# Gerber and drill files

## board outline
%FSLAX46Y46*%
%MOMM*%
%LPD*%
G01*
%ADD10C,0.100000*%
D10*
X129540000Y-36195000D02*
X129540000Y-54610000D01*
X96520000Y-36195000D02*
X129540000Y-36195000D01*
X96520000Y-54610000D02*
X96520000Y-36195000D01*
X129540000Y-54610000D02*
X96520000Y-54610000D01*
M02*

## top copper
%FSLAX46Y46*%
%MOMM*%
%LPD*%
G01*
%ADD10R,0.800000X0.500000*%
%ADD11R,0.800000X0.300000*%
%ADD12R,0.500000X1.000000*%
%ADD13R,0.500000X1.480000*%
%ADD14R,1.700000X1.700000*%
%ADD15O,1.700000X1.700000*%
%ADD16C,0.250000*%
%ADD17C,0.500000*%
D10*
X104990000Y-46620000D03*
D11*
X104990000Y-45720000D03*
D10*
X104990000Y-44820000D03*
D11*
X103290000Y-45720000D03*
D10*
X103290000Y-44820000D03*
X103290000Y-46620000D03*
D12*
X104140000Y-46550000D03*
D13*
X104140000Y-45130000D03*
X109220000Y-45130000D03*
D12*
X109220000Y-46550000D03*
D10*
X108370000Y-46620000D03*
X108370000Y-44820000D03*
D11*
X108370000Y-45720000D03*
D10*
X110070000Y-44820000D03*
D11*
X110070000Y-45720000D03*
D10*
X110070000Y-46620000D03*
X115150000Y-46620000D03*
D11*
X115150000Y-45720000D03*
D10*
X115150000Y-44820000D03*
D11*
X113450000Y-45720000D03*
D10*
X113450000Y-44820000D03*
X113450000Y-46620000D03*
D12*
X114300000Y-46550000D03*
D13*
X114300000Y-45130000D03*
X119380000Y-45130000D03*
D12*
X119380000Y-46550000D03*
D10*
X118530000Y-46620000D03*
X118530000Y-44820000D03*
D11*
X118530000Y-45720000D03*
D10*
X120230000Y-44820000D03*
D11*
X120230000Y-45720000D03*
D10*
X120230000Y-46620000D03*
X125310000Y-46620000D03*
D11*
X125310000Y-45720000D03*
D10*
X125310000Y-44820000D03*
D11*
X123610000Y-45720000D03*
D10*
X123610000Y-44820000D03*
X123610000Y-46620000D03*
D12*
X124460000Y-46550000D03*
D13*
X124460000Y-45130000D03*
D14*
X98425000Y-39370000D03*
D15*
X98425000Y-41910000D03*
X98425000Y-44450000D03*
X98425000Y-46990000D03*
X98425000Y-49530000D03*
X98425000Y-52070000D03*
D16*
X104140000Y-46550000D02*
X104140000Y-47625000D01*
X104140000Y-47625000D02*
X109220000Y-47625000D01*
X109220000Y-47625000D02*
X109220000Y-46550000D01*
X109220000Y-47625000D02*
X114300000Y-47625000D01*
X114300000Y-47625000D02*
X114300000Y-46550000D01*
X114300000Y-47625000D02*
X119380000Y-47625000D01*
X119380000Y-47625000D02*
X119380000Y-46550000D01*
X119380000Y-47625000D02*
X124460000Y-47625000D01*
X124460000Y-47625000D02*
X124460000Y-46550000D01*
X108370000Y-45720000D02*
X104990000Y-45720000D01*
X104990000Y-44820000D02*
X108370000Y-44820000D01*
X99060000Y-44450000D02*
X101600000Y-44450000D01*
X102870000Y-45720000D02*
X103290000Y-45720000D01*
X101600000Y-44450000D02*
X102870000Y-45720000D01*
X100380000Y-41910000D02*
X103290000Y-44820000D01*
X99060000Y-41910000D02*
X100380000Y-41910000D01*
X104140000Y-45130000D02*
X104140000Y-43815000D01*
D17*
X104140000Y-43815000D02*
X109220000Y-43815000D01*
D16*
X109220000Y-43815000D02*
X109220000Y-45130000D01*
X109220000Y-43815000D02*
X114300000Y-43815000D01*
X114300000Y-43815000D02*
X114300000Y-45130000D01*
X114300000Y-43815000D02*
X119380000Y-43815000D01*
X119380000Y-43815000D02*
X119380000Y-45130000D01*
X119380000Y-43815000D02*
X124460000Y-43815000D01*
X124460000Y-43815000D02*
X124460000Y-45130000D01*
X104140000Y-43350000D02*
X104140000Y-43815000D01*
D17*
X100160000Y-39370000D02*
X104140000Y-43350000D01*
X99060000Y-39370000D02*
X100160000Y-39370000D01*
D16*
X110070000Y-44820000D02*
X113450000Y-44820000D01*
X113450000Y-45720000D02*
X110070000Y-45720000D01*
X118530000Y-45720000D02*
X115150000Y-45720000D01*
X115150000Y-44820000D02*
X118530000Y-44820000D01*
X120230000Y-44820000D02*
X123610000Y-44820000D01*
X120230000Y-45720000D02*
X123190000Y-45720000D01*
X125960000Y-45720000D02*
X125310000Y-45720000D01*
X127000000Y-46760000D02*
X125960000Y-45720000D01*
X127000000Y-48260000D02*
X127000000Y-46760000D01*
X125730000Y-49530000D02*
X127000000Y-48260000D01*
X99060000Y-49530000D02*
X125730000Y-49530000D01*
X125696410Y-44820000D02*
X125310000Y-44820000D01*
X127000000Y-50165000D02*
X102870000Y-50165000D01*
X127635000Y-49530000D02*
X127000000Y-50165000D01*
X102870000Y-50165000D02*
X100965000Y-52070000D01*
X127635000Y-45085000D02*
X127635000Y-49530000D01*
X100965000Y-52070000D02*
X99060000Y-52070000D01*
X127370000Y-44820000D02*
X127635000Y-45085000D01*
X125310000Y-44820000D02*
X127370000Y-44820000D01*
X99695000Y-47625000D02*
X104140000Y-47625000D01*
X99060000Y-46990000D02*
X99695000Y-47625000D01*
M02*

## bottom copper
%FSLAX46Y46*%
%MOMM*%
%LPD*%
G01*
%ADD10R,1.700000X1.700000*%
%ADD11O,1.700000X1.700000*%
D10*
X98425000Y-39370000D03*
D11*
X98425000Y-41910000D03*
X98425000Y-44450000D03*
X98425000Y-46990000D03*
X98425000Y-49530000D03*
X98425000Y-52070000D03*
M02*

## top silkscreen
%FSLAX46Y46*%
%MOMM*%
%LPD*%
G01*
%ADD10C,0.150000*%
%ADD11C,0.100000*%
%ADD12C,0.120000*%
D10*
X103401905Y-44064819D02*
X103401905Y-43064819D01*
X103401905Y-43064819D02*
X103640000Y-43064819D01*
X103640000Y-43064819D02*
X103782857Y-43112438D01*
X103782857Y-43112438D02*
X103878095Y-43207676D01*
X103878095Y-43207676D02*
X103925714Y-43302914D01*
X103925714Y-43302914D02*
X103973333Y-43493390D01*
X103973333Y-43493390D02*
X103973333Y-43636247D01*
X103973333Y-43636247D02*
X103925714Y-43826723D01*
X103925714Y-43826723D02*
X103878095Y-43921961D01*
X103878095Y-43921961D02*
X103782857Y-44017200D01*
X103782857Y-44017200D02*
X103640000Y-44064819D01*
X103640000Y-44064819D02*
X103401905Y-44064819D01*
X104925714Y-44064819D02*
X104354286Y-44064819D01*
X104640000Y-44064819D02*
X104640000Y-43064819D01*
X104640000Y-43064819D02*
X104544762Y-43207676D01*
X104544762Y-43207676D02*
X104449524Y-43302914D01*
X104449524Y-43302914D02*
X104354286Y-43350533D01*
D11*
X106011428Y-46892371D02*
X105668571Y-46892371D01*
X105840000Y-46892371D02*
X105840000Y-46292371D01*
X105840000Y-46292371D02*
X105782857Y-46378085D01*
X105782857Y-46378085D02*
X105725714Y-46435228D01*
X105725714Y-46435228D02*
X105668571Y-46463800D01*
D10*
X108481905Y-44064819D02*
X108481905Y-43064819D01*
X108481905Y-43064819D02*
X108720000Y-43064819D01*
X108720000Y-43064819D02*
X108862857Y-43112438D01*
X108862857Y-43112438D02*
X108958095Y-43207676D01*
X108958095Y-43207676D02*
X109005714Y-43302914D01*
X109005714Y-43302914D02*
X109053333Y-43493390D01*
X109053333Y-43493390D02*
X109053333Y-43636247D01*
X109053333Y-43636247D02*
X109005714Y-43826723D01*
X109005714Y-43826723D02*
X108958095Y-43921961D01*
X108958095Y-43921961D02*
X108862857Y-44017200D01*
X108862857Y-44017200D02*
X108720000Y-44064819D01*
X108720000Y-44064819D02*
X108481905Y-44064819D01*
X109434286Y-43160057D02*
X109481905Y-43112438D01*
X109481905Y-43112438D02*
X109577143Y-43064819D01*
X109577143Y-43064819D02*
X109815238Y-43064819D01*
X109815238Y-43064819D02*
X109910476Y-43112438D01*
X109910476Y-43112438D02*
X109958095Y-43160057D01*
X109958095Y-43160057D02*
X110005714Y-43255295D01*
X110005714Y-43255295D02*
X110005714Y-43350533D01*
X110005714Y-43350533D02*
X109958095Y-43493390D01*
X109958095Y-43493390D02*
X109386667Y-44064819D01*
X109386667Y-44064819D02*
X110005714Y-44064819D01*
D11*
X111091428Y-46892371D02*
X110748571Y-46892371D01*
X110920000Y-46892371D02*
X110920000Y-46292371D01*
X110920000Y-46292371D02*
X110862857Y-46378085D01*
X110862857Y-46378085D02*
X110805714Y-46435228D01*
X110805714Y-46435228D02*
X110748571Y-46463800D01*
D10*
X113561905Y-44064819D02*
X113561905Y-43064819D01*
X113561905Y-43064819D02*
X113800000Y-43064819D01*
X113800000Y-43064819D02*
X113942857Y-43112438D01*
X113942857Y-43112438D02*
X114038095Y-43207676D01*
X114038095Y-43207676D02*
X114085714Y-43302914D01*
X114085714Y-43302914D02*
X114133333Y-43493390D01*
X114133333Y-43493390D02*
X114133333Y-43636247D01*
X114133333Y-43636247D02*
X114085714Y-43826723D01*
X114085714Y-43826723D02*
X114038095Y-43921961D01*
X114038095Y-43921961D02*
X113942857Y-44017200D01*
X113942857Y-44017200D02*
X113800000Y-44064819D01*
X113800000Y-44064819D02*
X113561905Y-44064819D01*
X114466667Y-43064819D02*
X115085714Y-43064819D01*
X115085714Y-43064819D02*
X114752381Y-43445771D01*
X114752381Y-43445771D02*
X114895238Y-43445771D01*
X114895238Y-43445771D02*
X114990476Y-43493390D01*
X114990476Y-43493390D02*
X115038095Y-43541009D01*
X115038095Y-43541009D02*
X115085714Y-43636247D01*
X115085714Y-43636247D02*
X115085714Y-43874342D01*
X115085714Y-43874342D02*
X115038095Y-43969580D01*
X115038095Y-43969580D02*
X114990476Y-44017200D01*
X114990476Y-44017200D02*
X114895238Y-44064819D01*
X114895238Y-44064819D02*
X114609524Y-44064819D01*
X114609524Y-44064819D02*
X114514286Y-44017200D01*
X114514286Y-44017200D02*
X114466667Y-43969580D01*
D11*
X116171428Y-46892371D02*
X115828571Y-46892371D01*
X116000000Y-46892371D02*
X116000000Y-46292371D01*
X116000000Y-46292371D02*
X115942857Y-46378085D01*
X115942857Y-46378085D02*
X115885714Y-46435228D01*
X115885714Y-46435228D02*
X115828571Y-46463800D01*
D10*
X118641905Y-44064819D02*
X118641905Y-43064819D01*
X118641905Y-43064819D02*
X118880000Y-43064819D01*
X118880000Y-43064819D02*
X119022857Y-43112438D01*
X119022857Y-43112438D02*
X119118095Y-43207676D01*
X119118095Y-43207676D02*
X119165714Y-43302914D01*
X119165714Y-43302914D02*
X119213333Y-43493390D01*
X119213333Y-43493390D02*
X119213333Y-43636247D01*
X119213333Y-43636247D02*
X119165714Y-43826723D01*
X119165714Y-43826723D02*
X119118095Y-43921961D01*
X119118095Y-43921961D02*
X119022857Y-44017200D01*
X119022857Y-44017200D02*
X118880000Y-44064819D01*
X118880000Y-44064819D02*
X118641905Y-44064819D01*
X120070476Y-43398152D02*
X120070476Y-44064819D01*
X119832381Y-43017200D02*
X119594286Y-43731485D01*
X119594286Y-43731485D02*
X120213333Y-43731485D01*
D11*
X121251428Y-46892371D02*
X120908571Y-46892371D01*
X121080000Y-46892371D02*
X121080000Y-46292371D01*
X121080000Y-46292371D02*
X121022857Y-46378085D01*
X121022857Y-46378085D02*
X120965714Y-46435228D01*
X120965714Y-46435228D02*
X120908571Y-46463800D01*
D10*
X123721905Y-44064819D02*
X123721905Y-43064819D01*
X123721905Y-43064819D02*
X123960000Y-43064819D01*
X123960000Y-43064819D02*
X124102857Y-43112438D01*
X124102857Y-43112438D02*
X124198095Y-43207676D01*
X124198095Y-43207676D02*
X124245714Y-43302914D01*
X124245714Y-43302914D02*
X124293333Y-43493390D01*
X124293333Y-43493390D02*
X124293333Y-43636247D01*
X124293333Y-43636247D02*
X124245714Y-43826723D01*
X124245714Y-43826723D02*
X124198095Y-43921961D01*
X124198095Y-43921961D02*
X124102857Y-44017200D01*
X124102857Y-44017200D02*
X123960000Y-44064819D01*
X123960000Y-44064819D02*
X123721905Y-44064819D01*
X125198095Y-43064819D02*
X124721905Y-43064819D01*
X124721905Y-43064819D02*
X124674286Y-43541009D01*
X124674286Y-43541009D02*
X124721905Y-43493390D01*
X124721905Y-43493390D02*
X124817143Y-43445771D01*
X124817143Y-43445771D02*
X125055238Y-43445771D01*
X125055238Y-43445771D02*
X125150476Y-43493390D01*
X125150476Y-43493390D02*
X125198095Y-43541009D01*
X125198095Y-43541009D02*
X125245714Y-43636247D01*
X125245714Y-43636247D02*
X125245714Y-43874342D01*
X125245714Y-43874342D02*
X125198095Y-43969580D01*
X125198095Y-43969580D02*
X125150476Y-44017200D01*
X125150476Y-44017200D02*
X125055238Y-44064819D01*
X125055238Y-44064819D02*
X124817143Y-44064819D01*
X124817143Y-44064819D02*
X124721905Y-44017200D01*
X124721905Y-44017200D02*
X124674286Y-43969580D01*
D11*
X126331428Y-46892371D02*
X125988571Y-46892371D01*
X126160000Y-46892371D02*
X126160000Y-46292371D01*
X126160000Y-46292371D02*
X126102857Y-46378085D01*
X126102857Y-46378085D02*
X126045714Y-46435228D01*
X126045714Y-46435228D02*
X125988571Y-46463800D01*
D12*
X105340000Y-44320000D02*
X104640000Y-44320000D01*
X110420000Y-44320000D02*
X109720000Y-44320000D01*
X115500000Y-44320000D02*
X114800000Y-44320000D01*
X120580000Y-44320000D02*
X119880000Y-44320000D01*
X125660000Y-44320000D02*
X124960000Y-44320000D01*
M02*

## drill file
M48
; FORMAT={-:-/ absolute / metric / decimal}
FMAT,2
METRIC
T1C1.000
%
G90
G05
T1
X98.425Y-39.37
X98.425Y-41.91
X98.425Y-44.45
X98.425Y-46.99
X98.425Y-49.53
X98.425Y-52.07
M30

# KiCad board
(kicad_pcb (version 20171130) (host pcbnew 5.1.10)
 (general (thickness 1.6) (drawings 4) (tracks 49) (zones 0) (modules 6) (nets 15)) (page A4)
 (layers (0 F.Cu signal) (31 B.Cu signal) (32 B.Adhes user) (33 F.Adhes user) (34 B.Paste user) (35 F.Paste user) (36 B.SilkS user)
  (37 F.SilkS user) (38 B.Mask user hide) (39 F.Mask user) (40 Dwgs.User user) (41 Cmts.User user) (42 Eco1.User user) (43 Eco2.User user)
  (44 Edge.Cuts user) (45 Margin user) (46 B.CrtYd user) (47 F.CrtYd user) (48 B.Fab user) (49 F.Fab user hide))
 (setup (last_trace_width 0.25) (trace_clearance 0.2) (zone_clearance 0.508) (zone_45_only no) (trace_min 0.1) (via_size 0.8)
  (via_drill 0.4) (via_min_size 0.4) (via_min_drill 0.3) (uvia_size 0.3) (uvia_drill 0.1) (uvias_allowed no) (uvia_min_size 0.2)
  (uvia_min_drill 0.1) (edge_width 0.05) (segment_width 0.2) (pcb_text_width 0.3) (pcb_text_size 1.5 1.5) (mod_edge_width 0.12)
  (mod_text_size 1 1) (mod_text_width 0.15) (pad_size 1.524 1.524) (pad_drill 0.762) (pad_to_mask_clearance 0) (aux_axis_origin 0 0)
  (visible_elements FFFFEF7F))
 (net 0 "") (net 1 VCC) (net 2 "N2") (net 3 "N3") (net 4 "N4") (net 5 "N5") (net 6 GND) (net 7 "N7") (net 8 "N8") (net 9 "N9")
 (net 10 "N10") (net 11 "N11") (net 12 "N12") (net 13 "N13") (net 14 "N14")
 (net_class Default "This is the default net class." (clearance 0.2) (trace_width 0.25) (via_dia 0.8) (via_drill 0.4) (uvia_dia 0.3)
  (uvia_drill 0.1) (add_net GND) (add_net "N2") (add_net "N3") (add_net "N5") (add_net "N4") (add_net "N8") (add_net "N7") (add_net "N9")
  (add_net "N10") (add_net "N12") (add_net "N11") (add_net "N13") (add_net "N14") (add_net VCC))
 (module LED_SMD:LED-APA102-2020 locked (layer F.Cu) (at 104.14 45.72 180)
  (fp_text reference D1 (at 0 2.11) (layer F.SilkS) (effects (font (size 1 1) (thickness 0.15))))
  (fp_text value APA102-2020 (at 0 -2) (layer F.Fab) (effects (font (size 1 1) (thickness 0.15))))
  (fp_line (start -1.2 1.4) (end -0.5 1.4) (layer F.SilkS) (width 0.12))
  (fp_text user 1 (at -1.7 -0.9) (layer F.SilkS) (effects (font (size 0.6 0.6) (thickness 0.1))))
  (pad 1 smd rect (at -0.85 -0.9 180) (size 0.8 0.5) (layers F.Cu F.Paste F.Mask) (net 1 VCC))
  (pad 2 smd rect (at -0.85 0 180) (size 0.8 0.3) (layers F.Cu F.Paste F.Mask) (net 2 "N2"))
  (pad 3 smd rect (at -0.85 0.9 180) (size 0.8 0.5) (layers F.Cu F.Paste F.Mask) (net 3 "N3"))
  (pad 5 smd rect (at 0.85 0 180) (size 0.8 0.3) (layers F.Cu F.Paste F.Mask) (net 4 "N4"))
  (pad 4 smd rect (at 0.85 0.9 180) (size 0.8 0.5) (layers F.Cu F.Paste F.Mask) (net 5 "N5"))
  (pad 6 smd rect (at 0.85 -0.9 180) (size 0.8 0.5) (layers F.Cu F.Paste F.Mask) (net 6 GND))
  (pad 1 smd rect (at 0 -0.83 270) (size 1 0.5) (layers F.Cu F.Paste F.Mask) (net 1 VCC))
  (pad 6 smd rect (at 0 0.59 270) (size 1.48 0.5) (layers F.Cu F.Paste F.Mask) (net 6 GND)))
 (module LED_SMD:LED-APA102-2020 (layer F.Cu) (at 109.22 45.72 180)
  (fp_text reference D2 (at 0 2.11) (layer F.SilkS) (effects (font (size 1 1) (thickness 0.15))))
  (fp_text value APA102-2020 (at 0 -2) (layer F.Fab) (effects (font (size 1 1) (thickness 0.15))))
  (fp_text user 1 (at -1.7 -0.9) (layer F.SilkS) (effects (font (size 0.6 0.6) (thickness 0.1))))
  (fp_line (start -1.2 1.4) (end -0.5 1.4) (layer F.SilkS) (width 0.12))
  (pad 6 smd rect (at 0 0.59 270) (size 1.48 0.5) (layers F.Cu F.Paste F.Mask) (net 6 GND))
  (pad 1 smd rect (at 0 -0.83 270) (size 1 0.5) (layers F.Cu F.Paste F.Mask) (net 1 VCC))
  (pad 6 smd rect (at 0.85 -0.9 180) (size 0.8 0.5) (layers F.Cu F.Paste F.Mask) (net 6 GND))
  (pad 4 smd rect (at 0.85 0.9 180) (size 0.8 0.5) (layers F.Cu F.Paste F.Mask) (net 3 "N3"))
  (pad 5 smd rect (at 0.85 0 180) (size 0.8 0.3) (layers F.Cu F.Paste F.Mask) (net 2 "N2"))
  (pad 3 smd rect (at -0.85 0.9 180) (size 0.8 0.5) (layers F.Cu F.Paste F.Mask) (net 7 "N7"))
  (pad 2 smd rect (at -0.85 0 180) (size 0.8 0.3) (layers F.Cu F.Paste F.Mask) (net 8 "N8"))
  (pad 1 smd rect (at -0.85 -0.9 180) (size 0.8 0.5) (layers F.Cu F.Paste F.Mask) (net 1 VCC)))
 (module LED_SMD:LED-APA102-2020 (layer F.Cu) (at 114.3 45.72 180)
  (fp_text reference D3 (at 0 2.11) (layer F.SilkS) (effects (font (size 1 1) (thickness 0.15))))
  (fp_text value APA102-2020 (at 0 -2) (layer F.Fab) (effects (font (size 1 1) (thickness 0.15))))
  (fp_line (start -1.2 1.4) (end -0.5 1.4) (layer F.SilkS) (width 0.12))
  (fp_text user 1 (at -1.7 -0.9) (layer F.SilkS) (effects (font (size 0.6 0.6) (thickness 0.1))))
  (pad 1 smd rect (at -0.85 -0.9 180) (size 0.8 0.5) (layers F.Cu F.Paste F.Mask) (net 1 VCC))
  (pad 2 smd rect (at -0.85 0 180) (size 0.8 0.3) (layers F.Cu F.Paste F.Mask) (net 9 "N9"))
  (pad 3 smd rect (at -0.85 0.9 180) (size 0.8 0.5) (layers F.Cu F.Paste F.Mask) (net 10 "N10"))
  (pad 5 smd rect (at 0.85 0 180) (size 0.8 0.3) (layers F.Cu F.Paste F.Mask) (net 8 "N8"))
  (pad 4 smd rect (at 0.85 0.9 180) (size 0.8 0.5) (layers F.Cu F.Paste F.Mask) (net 7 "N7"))
  (pad 6 smd rect (at 0.85 -0.9 180) (size 0.8 0.5) (layers F.Cu F.Paste F.Mask) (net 6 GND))
  (pad 1 smd rect (at 0 -0.83 270) (size 1 0.5) (layers F.Cu F.Paste F.Mask) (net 1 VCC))
  (pad 6 smd rect (at 0 0.59 270) (size 1.48 0.5) (layers F.Cu F.Paste F.Mask) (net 6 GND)))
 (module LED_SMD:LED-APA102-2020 (layer F.Cu) (at 119.38 45.72 180)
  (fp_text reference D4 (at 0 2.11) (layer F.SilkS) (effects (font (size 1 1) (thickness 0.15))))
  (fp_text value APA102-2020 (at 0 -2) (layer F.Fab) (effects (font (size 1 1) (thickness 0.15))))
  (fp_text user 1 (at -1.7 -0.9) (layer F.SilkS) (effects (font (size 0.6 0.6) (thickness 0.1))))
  (fp_line (start -1.2 1.4) (end -0.5 1.4) (layer F.SilkS) (width 0.12))
  (pad 6 smd rect (at 0 0.59 270) (size 1.48 0.5) (layers F.Cu F.Paste F.Mask) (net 6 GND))
  (pad 1 smd rect (at 0 -0.83 270) (size 1 0.5) (layers F.Cu F.Paste F.Mask) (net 1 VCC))
  (pad 6 smd rect (at 0.85 -0.9 180) (size 0.8 0.5) (layers F.Cu F.Paste F.Mask) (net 6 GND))
  (pad 4 smd rect (at 0.85 0.9 180) (size 0.8 0.5) (layers F.Cu F.Paste F.Mask) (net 10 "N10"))
  (pad 5 smd rect (at 0.85 0 180) (size 0.8 0.3) (layers F.Cu F.Paste F.Mask) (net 9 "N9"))
  (pad 3 smd rect (at -0.85 0.9 180) (size 0.8 0.5) (layers F.Cu F.Paste F.Mask) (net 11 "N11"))
  (pad 2 smd rect (at -0.85 0 180) (size 0.8 0.3) (layers F.Cu F.Paste F.Mask) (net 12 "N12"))
  (pad 1 smd rect (at -0.85 -0.9 180) (size 0.8 0.5) (layers F.Cu F.Paste F.Mask) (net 1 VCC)))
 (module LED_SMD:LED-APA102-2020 (layer F.Cu) (at 124.46 45.72 180)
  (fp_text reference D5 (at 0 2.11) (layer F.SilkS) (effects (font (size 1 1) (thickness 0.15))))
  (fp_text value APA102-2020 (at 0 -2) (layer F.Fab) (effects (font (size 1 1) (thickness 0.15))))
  (fp_line (start -1.2 1.4) (end -0.5 1.4) (layer F.SilkS) (width 0.12))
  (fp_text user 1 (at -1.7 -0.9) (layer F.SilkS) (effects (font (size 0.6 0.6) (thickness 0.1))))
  (pad 1 smd rect (at -0.85 -0.9 180) (size 0.8 0.5) (layers F.Cu F.Paste F.Mask) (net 1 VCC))
  (pad 2 smd rect (at -0.85 0 180) (size 0.8 0.3) (layers F.Cu F.Paste F.Mask) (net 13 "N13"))
  (pad 3 smd rect (at -0.85 0.9 180) (size 0.8 0.5) (layers F.Cu F.Paste F.Mask) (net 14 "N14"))
  (pad 5 smd rect (at 0.85 0 180) (size 0.8 0.3) (layers F.Cu F.Paste F.Mask) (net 12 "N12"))
  (pad 4 smd rect (at 0.85 0.9 180) (size 0.8 0.5) (layers F.Cu F.Paste F.Mask) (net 11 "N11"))
  (pad 6 smd rect (at 0.85 -0.9 180) (size 0.8 0.5) (layers F.Cu F.Paste F.Mask) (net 6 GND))
  (pad 1 smd rect (at 0 -0.83 270) (size 1 0.5) (layers F.Cu F.Paste F.Mask) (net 1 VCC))
  (pad 6 smd rect (at 0 0.59 270) (size 1.48 0.5) (layers F.Cu F.Paste F.Mask) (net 6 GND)))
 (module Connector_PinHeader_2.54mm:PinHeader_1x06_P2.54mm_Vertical (layer B.Cu) (at 98.425 39.37 180)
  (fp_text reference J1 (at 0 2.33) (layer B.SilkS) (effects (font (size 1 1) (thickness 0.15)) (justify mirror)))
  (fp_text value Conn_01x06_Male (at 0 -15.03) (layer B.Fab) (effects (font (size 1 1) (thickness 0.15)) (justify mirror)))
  (pad 1 thru_hole rect (at 0 0 180) (size 1.7 1.7) (drill 1) (layers *.Cu *.Mask) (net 6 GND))
  (pad 2 thru_hole oval (at 0 -2.54 180) (size 1.7 1.7) (drill 1) (layers *.Cu *.Mask) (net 5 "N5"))
  (pad 3 thru_hole oval (at 0 -5.08 180) (size 1.7 1.7) (drill 1) (layers *.Cu *.Mask) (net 4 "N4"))
  (pad 4 thru_hole oval (at 0 -7.62 180) (size 1.7 1.7) (drill 1) (layers *.Cu *.Mask) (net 1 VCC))
  (pad 5 thru_hole oval (at 0 -10.16 180) (size 1.7 1.7) (drill 1) (layers *.Cu *.Mask) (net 13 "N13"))
  (pad 6 thru_hole oval (at 0 -12.7 180) (size 1.7 1.7) (drill 1) (layers *.Cu *.Mask) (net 14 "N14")))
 (gr_line (start 129.54 36.195) (end 129.54 54.61) (layer Edge.Cuts) (width 0.1))
 (gr_line (start 96.52 36.195) (end 129.54 36.195) (layer Edge.Cuts) (width 0.1))
 (gr_line (start 96.52 54.61) (end 96.52 36.195) (layer Edge.Cuts) (width 0.1))
 (gr_line (start 129.54 54.61) (end 96.52 54.61) (layer Edge.Cuts) (width 0.1))
 (segment (start 104.14 46.55) (end 104.14 47.625) (width 0.25) (layer F.Cu) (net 1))
 (segment (start 104.14 47.625) (end 109.22 47.625) (width 0.25) (layer F.Cu) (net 1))
 (segment (start 109.22 47.625) (end 109.22 46.55) (width 0.25) (layer F.Cu) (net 1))
 (segment (start 109.22 47.625) (end 114.3 47.625) (width 0.25) (layer F.Cu) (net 1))
 (segment (start 114.3 47.625) (end 114.3 46.55) (width 0.25) (layer F.Cu) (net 1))
 (segment (start 114.3 47.625) (end 119.38 47.625) (width 0.25) (layer F.Cu) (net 1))
 (segment (start 119.38 47.625) (end 119.38 46.55) (width 0.25) (layer F.Cu) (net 1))
 (segment (start 119.38 47.625) (end 124.46 47.625) (width 0.25) (layer F.Cu) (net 1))
 (segment (start 124.46 47.625) (end 124.46 46.55) (width 0.25) (layer F.Cu) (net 1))
 (segment (start 108.37 45.72) (end 104.99 45.72) (width 0.25) (layer F.Cu) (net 2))
 (segment (start 104.99 44.82) (end 108.37 44.82) (width 0.25) (layer F.Cu) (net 3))
 (segment (start 99.06 44.45) (end 101.6 44.45) (width 0.25) (layer F.Cu) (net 4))
 (segment (start 102.87 45.72) (end 103.29 45.72) (width 0.25) (layer F.Cu) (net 4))
 (segment (start 101.6 44.45) (end 102.87 45.72) (width 0.25) (layer F.Cu) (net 4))
 (segment (start 100.38 41.91) (end 103.29 44.82) (width 0.25) (layer F.Cu) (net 5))
 (segment (start 99.06 41.91) (end 100.38 41.91) (width 0.25) (layer F.Cu) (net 5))
 (segment (start 104.14 45.13) (end 104.14 43.815) (width 0.25) (layer F.Cu) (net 6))
 (segment (start 104.14 43.815) (end 109.22 43.815) (width 0.5) (layer F.Cu) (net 6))
 (segment (start 109.22 43.815) (end 109.22 45.13) (width 0.25) (layer F.Cu) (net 6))
 (segment (start 109.22 43.815) (end 114.3 43.815) (width 0.25) (layer F.Cu) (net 6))
 (segment (start 114.3 43.815) (end 114.3 45.13) (width 0.25) (layer F.Cu) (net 6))
 (segment (start 114.3 43.815) (end 119.38 43.815) (width 0.25) (layer F.Cu) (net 6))
 (segment (start 119.38 43.815) (end 119.38 45.13) (width 0.25) (layer F.Cu) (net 6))
 (segment (start 119.38 43.815) (end 124.46 43.815) (width 0.25) (layer F.Cu) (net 6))
 (segment (start 124.46 43.815) (end 124.46 45.13) (width 0.25) (layer F.Cu) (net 6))
 (segment (start 104.14 43.35) (end 104.14 43.815) (width 0.25) (layer F.Cu) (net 6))
 (segment (start 100.16 39.37) (end 104.14 43.35) (width 0.5) (layer F.Cu) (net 6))
 (segment (start 99.06 39.37) (end 100.16 39.37) (width 0.5) (layer F.Cu) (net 6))
 (segment (start 110.07 44.82) (end 113.45 44.82) (width 0.25) (layer F.Cu) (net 7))
 (segment (start 113.45 45.72) (end 110.07 45.72) (width 0.25) (layer F.Cu) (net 8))
 (segment (start 118.53 45.72) (end 115.15 45.72) (width 0.25) (layer F.Cu) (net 9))
 (segment (start 115.15 44.82) (end 118.53 44.82) (width 0.25) (layer F.Cu) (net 10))
 (segment (start 120.23 44.82) (end 123.61 44.82) (width 0.25) (layer F.Cu) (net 11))
 (segment (start 120.23 45.72) (end 123.19 45.72) (width 0.25) (layer F.Cu) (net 12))
 (segment (start 125.96 45.72) (end 125.31 45.72) (width 0.25) (layer F.Cu) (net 13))
 (segment (start 127 46.76) (end 125.96 45.72) (width 0.25) (layer F.Cu) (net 13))
 (segment (start 127 48.26) (end 127 46.76) (width 0.25) (layer F.Cu) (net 13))
 (segment (start 125.73 49.53) (end 127 48.26) (width 0.25) (layer F.Cu) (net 13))
 (segment (start 99.06 49.53) (end 125.73 49.53) (width 0.25) (layer F.Cu) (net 13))
 (segment (start 125.69641 44.82) (end 125.31 44.82) (width 0.25) (layer F.Cu) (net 14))
 (segment (start 127 50.165) (end 102.87 50.165) (width 0.25) (layer F.Cu) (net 14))
 (segment (start 127.635 49.53) (end 127 50.165) (width 0.25) (layer F.Cu) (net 14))
 (segment (start 102.87 50.165) (end 100.965 52.07) (width 0.25) (layer F.Cu) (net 14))
 (segment (start 127.635 45.085) (end 127.635 49.53) (width 0.25) (layer F.Cu) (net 14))
 (segment (start 100.965 52.07) (end 99.06 52.07) (width 0.25) (layer F.Cu) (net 14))
 (segment (start 127.37 44.82) (end 127.635 45.085) (width 0.25) (layer F.Cu) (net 14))
 (segment (start 125.31 44.82) (end 127.37 44.82) (width 0.25) (layer F.Cu) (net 14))
 (segment (start 99.695 47.625) (end 104.14 47.625) (width 0.25) (layer F.Cu) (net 1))
 (segment (start 99.06 46.99) (end 99.695 47.625) (width 0.25) (layer F.Cu) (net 1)))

